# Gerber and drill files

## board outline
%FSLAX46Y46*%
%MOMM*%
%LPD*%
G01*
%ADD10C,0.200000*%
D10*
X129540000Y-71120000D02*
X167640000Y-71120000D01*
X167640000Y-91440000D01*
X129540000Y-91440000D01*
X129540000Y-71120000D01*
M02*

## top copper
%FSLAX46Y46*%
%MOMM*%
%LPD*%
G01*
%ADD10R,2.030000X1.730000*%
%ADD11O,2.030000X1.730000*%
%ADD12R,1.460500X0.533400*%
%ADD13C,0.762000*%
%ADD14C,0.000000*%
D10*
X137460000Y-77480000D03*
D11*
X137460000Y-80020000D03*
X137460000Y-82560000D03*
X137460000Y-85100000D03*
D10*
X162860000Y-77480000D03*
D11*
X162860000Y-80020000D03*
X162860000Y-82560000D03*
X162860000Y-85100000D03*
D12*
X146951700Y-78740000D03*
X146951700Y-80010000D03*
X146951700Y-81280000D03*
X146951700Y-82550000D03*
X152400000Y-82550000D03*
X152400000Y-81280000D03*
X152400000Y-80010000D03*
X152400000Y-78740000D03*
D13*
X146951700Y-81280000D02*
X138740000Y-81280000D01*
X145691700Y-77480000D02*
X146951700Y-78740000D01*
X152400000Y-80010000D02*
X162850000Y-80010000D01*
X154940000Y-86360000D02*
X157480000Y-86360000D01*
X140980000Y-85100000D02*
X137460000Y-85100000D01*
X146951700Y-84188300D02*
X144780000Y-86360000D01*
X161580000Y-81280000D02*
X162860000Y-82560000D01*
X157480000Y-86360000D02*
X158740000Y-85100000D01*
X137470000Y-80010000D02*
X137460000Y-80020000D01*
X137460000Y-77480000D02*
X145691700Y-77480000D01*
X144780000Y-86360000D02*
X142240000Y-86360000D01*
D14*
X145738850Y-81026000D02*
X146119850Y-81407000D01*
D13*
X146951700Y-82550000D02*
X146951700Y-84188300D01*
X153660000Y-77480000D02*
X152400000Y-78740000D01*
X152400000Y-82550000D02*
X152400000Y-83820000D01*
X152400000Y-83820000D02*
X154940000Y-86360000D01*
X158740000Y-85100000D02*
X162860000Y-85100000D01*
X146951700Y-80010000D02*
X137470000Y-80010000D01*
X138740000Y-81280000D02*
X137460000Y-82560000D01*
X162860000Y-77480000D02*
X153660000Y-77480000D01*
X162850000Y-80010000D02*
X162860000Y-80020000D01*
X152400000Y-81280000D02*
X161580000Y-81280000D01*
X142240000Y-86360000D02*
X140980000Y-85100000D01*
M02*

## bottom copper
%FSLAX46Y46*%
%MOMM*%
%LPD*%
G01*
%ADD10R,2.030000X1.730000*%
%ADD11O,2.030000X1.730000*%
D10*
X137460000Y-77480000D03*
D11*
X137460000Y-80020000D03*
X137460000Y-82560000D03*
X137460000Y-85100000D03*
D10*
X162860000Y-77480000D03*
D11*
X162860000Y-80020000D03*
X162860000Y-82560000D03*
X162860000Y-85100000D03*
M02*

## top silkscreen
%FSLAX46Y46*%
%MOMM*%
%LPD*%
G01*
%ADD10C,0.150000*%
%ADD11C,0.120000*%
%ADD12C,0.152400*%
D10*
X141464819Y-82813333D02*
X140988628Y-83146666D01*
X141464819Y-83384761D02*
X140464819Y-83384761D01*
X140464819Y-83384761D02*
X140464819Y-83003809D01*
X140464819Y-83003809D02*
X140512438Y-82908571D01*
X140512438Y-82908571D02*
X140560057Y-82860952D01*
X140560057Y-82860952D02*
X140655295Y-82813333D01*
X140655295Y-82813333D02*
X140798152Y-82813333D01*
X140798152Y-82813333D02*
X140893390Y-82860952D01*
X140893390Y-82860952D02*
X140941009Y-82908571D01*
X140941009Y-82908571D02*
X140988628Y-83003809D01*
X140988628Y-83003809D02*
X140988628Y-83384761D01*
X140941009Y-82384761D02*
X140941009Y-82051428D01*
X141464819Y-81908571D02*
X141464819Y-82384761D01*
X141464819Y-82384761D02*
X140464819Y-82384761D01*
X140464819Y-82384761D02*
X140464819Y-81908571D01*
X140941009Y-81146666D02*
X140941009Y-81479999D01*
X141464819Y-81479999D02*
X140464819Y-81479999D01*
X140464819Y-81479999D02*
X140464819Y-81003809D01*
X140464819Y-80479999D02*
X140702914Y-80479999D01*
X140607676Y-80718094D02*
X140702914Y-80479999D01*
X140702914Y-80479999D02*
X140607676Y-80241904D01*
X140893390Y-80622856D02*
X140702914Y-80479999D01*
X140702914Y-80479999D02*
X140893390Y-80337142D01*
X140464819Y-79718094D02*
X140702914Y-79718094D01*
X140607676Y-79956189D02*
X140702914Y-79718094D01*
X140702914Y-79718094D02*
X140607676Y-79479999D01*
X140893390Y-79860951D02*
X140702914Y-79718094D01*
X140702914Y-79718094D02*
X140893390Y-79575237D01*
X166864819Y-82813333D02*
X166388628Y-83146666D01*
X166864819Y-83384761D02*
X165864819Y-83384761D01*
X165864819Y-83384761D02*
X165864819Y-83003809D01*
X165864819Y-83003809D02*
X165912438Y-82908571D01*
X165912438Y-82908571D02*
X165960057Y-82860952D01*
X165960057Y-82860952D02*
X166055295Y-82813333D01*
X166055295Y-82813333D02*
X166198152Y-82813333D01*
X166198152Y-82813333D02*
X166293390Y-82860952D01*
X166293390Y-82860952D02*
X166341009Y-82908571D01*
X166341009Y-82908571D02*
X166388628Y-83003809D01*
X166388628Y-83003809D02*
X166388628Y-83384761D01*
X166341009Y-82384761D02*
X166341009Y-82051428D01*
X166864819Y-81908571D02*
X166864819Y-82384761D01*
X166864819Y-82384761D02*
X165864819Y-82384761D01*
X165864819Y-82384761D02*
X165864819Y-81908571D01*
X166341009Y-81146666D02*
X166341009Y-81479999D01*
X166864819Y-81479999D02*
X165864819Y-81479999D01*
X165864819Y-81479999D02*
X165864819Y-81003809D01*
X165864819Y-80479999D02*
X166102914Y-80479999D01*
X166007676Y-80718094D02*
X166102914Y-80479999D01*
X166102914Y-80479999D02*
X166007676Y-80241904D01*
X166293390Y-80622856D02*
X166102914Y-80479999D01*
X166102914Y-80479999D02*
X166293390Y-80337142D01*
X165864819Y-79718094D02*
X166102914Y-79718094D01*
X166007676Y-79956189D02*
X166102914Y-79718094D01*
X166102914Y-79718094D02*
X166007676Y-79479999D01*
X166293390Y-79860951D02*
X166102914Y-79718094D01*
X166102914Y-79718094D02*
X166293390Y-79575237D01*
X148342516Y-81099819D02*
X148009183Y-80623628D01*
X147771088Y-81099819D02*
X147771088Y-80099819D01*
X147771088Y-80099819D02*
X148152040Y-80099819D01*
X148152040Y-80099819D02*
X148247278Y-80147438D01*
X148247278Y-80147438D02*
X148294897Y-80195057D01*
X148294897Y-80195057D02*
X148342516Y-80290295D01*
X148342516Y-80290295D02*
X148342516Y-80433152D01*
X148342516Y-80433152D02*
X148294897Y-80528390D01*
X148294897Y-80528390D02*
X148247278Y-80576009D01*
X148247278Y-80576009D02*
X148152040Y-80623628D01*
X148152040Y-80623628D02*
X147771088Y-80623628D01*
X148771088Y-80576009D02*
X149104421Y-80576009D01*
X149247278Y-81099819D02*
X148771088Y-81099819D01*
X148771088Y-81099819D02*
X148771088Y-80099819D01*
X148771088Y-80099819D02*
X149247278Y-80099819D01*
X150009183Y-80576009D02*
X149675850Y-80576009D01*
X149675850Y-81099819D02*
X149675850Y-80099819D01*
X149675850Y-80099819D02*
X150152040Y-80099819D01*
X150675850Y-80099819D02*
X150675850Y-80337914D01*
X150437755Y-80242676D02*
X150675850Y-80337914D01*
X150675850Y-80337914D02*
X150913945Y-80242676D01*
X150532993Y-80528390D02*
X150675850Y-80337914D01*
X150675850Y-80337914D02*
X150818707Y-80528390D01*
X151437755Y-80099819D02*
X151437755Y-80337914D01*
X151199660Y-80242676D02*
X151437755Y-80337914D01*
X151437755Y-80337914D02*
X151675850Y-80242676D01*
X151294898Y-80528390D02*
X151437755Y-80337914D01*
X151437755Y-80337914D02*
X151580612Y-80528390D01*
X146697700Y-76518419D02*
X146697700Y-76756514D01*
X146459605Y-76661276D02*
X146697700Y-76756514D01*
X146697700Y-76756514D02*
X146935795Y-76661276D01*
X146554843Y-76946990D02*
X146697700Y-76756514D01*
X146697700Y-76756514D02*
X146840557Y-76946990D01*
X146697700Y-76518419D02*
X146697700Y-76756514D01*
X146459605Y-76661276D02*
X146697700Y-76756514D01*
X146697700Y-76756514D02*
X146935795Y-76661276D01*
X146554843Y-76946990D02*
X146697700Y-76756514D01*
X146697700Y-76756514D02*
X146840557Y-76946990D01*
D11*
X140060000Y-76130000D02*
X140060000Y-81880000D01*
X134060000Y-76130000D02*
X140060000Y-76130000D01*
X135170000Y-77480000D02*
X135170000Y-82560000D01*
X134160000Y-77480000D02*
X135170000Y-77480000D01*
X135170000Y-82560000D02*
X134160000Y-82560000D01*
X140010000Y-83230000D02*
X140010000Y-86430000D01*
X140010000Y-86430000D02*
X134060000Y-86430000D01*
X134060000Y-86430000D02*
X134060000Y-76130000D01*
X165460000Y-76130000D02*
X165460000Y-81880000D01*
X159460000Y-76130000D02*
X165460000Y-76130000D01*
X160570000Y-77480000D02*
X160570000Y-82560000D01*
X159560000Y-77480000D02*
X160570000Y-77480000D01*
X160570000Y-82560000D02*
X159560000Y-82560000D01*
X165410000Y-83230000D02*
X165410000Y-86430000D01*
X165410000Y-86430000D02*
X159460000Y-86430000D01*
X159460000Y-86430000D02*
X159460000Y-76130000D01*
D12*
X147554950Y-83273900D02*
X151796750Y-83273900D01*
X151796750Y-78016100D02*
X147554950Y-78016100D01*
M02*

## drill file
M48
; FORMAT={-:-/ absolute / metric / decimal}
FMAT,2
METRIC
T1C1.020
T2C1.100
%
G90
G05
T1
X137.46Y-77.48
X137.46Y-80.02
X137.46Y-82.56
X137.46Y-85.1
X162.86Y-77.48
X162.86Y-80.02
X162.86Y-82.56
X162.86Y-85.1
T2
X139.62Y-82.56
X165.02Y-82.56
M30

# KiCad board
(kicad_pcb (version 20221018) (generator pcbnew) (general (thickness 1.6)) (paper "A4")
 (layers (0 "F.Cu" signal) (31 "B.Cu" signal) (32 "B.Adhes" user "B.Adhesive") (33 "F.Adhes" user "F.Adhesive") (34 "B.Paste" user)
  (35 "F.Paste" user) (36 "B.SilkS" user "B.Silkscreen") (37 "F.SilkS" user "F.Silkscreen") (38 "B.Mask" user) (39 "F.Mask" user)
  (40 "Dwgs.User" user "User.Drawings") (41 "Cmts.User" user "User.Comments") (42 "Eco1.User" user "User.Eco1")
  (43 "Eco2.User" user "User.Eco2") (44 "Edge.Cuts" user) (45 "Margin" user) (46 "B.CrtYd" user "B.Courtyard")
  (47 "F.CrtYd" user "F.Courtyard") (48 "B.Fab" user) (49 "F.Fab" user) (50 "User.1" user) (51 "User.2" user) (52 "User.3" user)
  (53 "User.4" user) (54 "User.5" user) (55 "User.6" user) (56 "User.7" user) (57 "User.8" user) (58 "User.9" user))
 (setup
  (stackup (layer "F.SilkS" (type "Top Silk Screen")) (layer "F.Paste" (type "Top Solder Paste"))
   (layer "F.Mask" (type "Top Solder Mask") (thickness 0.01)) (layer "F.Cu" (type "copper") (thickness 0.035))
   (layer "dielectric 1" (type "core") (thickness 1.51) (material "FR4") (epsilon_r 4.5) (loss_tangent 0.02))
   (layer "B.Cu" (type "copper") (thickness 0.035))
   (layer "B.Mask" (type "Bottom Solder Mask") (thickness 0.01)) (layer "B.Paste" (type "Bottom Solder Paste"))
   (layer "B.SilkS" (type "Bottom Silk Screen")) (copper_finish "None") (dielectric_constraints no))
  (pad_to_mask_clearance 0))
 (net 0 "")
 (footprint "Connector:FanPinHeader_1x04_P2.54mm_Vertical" (layer "F.Cu") (at 137.46 77.48 -90)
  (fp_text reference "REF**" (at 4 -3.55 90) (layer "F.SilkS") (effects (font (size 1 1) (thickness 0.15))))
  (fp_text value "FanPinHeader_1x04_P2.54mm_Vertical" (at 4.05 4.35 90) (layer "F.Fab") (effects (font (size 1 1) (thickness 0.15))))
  (fp_line (start -1.35 -2.6) (end 4.4 -2.6) (stroke (width 0.12) (type solid)) (layer "F.SilkS"))
  (fp_line (start -1.35 3.4) (end -1.35 -2.6) (stroke (width 0.12) (type solid)) (layer "F.SilkS"))
  (fp_line (start 0 2.29) (end 5.08 2.29) (stroke (width 0.12) (type solid)) (layer "F.SilkS"))
  (fp_line (start 0 3.3) (end 0 2.29) (stroke (width 0.12) (type solid)) (layer "F.SilkS"))
  (fp_line (start 5.08 2.29) (end 5.08 3.3) (stroke (width 0.12) (type solid)) (layer "F.SilkS"))
  (fp_line (start 5.75 -2.55) (end 8.95 -2.55) (stroke (width 0.12) (type solid)) (layer "F.SilkS"))
  (fp_line (start 8.95 -2.55) (end 8.95 3.4) (stroke (width 0.12) (type solid)) (layer "F.SilkS"))
  (fp_line (start 8.95 3.4) (end -1.35 3.4) (stroke (width 0.12) (type solid)) (layer "F.SilkS"))
  (pad "" np_thru_hole circle (at 5.08 -2.16) (size 1.1 1.1) (drill 1.1) (layers "*.Cu" "*.Mask"))
  (pad "1" thru_hole rect (at 0 0) (size 2.03 1.73) (drill 1.02) (layers "*.Cu" "*.Mask"))
  (pad "2" thru_hole oval (at 2.54 0) (size 2.03 1.73) (drill 1.02) (layers "*.Cu" "*.Mask"))
  (pad "3" thru_hole oval (at 5.08 0) (size 2.03 1.73) (drill 1.02) (layers "*.Cu" "*.Mask"))
  (pad "4" thru_hole oval (at 7.62 0) (size 2.03 1.73) (drill 1.02) (layers "*.Cu" "*.Mask")))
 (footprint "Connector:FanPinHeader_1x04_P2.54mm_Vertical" (layer "F.Cu") (at 162.86 77.48 -90)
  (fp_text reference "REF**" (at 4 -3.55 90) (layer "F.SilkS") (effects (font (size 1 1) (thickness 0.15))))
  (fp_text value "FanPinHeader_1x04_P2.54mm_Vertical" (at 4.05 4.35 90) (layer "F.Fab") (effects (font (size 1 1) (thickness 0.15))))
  (fp_line (start -1.35 -2.6) (end 4.4 -2.6) (stroke (width 0.12) (type solid)) (layer "F.SilkS"))
  (fp_line (start -1.35 3.4) (end -1.35 -2.6) (stroke (width 0.12) (type solid)) (layer "F.SilkS"))
  (fp_line (start 0 2.29) (end 5.08 2.29) (stroke (width 0.12) (type solid)) (layer "F.SilkS"))
  (fp_line (start 0 3.3) (end 0 2.29) (stroke (width 0.12) (type solid)) (layer "F.SilkS"))
  (fp_line (start 5.08 2.29) (end 5.08 3.3) (stroke (width 0.12) (type solid)) (layer "F.SilkS"))
  (fp_line (start 5.75 -2.55) (end 8.95 -2.55) (stroke (width 0.12) (type solid)) (layer "F.SilkS"))
  (fp_line (start 8.95 -2.55) (end 8.95 3.4) (stroke (width 0.12) (type solid)) (layer "F.SilkS"))
  (fp_line (start 8.95 3.4) (end -1.35 3.4) (stroke (width 0.12) (type solid)) (layer "F.SilkS"))
  (pad "" np_thru_hole circle (at 5.08 -2.16) (size 1.1 1.1) (drill 1.1) (layers "*.Cu" "*.Mask"))
  (pad "1" thru_hole rect (at 0 0) (size 2.03 1.73) (drill 1.02) (layers "*.Cu" "*.Mask"))
  (pad "2" thru_hole oval (at 2.54 0) (size 2.03 1.73) (drill 1.02) (layers "*.Cu" "*.Mask"))
  (pad "3" thru_hole oval (at 5.08 0) (size 2.03 1.73) (drill 1.02) (layers "*.Cu" "*.Mask"))
  (pad "4" thru_hole oval (at 7.62 0) (size 2.03 1.73) (drill 1.02) (layers "*.Cu" "*.Mask")))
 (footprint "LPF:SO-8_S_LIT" (layer "F.Cu") (at 149.67585 80.645)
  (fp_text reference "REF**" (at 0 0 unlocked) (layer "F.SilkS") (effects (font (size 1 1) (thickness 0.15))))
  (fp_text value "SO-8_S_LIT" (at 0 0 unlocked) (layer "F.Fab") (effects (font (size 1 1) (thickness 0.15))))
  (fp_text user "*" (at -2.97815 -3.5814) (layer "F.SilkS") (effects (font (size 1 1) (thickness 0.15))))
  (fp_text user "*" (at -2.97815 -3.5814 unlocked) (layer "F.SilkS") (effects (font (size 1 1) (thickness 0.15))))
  (fp_line (start -2.1209 2.6289) (end 2.1209 2.6289) (stroke (width 0.1524) (type solid)) (layer "F.SilkS"))
  (fp_line (start 2.1209 -2.6289) (end -2.1209 -2.6289) (stroke (width 0.1524) (type solid)) (layer "F.SilkS"))
  (pad "1" smd rect (at -2.72415 -1.905) (size 1.4605 0.5334) (layers "F.Cu" "F.Paste" "F.Mask"))
  (pad "2" smd rect (at -2.72415 -0.635) (size 1.4605 0.5334) (layers "F.Cu" "F.Paste" "F.Mask"))
  (pad "3" smd rect (at -2.72415 0.635) (size 1.4605 0.5334) (layers "F.Cu" "F.Paste" "F.Mask"))
  (pad "4" smd rect (at -2.72415 1.905) (size 1.4605 0.5334) (layers "F.Cu" "F.Paste" "F.Mask"))
  (pad "5" smd rect (at 2.72415 1.905) (size 1.4605 0.5334) (layers "F.Cu" "F.Paste" "F.Mask"))
  (pad "6" smd rect (at 2.72415 0.635) (size 1.4605 0.5334) (layers "F.Cu" "F.Paste" "F.Mask"))
  (pad "7" smd rect (at 2.72415 -0.635) (size 1.4605 0.5334) (layers "F.Cu" "F.Paste" "F.Mask"))
  (pad "8" smd rect (at 2.72415 -1.905) (size 1.4605 0.5334) (layers "F.Cu" "F.Paste" "F.Mask")))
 (gr_rect (start 129.54 71.12) (end 167.64 91.44) (stroke (width 0.2) (type default)) (fill none) (layer "Edge.Cuts"))
 (segment (start 146.9517 81.28) (end 138.74 81.28) (width 0.762) (layer "F.Cu") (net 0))
 (segment (start 145.6917 77.48) (end 146.9517 78.74) (width 0.762) (layer "F.Cu") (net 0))
 (segment (start 152.4 80.01) (end 162.85 80.01) (width 0.762) (layer "F.Cu") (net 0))
 (segment (start 154.94 86.36) (end 157.48 86.36) (width 0.762) (layer "F.Cu") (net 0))
 (segment (start 140.98 85.1) (end 137.46 85.1) (width 0.762) (layer "F.Cu") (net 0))
 (segment (start 146.9517 84.1883) (end 144.78 86.36) (width 0.762) (layer "F.Cu") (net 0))
 (segment (start 161.58 81.28) (end 162.86 82.56) (width 0.762) (layer "F.Cu") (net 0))
 (segment (start 157.48 86.36) (end 158.74 85.1) (width 0.762) (layer "F.Cu") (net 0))
 (segment (start 137.47 80.01) (end 137.46 80.02) (width 0.762) (layer "F.Cu") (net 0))
 (segment (start 137.46 77.48) (end 145.6917 77.48) (width 0.762) (layer "F.Cu") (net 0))
 (segment (start 144.78 86.36) (end 142.24 86.36) (width 0.762) (layer "F.Cu") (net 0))
 (segment (start 145.73885 81.026) (end 146.11985 81.407) (width 0) (layer "F.Cu") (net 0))
 (segment (start 146.9517 82.55) (end 146.9517 84.1883) (width 0.762) (layer "F.Cu") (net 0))
 (segment (start 153.66 77.48) (end 152.4 78.74) (width 0.762) (layer "F.Cu") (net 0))
 (segment (start 152.4 82.55) (end 152.4 83.82) (width 0.762) (layer "F.Cu") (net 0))
 (segment (start 152.4 83.82) (end 154.94 86.36) (width 0.762) (layer "F.Cu") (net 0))
 (segment (start 158.74 85.1) (end 162.86 85.1) (width 0.762) (layer "F.Cu") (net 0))
 (segment (start 146.9517 80.01) (end 137.47 80.01) (width 0.762) (layer "F.Cu") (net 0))
 (segment (start 138.74 81.28) (end 137.46 82.56) (width 0.762) (layer "F.Cu") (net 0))
 (segment (start 162.86 77.48) (end 153.66 77.48) (width 0.762) (layer "F.Cu") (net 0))
 (segment (start 162.85 80.01) (end 162.86 80.02) (width 0.762) (layer "F.Cu") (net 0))
 (segment (start 152.4 81.28) (end 161.58 81.28) (width 0.762) (layer "F.Cu") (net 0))
 (segment (start 142.24 86.36) (end 140.98 85.1) (width 0.762) (layer "F.Cu") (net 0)))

